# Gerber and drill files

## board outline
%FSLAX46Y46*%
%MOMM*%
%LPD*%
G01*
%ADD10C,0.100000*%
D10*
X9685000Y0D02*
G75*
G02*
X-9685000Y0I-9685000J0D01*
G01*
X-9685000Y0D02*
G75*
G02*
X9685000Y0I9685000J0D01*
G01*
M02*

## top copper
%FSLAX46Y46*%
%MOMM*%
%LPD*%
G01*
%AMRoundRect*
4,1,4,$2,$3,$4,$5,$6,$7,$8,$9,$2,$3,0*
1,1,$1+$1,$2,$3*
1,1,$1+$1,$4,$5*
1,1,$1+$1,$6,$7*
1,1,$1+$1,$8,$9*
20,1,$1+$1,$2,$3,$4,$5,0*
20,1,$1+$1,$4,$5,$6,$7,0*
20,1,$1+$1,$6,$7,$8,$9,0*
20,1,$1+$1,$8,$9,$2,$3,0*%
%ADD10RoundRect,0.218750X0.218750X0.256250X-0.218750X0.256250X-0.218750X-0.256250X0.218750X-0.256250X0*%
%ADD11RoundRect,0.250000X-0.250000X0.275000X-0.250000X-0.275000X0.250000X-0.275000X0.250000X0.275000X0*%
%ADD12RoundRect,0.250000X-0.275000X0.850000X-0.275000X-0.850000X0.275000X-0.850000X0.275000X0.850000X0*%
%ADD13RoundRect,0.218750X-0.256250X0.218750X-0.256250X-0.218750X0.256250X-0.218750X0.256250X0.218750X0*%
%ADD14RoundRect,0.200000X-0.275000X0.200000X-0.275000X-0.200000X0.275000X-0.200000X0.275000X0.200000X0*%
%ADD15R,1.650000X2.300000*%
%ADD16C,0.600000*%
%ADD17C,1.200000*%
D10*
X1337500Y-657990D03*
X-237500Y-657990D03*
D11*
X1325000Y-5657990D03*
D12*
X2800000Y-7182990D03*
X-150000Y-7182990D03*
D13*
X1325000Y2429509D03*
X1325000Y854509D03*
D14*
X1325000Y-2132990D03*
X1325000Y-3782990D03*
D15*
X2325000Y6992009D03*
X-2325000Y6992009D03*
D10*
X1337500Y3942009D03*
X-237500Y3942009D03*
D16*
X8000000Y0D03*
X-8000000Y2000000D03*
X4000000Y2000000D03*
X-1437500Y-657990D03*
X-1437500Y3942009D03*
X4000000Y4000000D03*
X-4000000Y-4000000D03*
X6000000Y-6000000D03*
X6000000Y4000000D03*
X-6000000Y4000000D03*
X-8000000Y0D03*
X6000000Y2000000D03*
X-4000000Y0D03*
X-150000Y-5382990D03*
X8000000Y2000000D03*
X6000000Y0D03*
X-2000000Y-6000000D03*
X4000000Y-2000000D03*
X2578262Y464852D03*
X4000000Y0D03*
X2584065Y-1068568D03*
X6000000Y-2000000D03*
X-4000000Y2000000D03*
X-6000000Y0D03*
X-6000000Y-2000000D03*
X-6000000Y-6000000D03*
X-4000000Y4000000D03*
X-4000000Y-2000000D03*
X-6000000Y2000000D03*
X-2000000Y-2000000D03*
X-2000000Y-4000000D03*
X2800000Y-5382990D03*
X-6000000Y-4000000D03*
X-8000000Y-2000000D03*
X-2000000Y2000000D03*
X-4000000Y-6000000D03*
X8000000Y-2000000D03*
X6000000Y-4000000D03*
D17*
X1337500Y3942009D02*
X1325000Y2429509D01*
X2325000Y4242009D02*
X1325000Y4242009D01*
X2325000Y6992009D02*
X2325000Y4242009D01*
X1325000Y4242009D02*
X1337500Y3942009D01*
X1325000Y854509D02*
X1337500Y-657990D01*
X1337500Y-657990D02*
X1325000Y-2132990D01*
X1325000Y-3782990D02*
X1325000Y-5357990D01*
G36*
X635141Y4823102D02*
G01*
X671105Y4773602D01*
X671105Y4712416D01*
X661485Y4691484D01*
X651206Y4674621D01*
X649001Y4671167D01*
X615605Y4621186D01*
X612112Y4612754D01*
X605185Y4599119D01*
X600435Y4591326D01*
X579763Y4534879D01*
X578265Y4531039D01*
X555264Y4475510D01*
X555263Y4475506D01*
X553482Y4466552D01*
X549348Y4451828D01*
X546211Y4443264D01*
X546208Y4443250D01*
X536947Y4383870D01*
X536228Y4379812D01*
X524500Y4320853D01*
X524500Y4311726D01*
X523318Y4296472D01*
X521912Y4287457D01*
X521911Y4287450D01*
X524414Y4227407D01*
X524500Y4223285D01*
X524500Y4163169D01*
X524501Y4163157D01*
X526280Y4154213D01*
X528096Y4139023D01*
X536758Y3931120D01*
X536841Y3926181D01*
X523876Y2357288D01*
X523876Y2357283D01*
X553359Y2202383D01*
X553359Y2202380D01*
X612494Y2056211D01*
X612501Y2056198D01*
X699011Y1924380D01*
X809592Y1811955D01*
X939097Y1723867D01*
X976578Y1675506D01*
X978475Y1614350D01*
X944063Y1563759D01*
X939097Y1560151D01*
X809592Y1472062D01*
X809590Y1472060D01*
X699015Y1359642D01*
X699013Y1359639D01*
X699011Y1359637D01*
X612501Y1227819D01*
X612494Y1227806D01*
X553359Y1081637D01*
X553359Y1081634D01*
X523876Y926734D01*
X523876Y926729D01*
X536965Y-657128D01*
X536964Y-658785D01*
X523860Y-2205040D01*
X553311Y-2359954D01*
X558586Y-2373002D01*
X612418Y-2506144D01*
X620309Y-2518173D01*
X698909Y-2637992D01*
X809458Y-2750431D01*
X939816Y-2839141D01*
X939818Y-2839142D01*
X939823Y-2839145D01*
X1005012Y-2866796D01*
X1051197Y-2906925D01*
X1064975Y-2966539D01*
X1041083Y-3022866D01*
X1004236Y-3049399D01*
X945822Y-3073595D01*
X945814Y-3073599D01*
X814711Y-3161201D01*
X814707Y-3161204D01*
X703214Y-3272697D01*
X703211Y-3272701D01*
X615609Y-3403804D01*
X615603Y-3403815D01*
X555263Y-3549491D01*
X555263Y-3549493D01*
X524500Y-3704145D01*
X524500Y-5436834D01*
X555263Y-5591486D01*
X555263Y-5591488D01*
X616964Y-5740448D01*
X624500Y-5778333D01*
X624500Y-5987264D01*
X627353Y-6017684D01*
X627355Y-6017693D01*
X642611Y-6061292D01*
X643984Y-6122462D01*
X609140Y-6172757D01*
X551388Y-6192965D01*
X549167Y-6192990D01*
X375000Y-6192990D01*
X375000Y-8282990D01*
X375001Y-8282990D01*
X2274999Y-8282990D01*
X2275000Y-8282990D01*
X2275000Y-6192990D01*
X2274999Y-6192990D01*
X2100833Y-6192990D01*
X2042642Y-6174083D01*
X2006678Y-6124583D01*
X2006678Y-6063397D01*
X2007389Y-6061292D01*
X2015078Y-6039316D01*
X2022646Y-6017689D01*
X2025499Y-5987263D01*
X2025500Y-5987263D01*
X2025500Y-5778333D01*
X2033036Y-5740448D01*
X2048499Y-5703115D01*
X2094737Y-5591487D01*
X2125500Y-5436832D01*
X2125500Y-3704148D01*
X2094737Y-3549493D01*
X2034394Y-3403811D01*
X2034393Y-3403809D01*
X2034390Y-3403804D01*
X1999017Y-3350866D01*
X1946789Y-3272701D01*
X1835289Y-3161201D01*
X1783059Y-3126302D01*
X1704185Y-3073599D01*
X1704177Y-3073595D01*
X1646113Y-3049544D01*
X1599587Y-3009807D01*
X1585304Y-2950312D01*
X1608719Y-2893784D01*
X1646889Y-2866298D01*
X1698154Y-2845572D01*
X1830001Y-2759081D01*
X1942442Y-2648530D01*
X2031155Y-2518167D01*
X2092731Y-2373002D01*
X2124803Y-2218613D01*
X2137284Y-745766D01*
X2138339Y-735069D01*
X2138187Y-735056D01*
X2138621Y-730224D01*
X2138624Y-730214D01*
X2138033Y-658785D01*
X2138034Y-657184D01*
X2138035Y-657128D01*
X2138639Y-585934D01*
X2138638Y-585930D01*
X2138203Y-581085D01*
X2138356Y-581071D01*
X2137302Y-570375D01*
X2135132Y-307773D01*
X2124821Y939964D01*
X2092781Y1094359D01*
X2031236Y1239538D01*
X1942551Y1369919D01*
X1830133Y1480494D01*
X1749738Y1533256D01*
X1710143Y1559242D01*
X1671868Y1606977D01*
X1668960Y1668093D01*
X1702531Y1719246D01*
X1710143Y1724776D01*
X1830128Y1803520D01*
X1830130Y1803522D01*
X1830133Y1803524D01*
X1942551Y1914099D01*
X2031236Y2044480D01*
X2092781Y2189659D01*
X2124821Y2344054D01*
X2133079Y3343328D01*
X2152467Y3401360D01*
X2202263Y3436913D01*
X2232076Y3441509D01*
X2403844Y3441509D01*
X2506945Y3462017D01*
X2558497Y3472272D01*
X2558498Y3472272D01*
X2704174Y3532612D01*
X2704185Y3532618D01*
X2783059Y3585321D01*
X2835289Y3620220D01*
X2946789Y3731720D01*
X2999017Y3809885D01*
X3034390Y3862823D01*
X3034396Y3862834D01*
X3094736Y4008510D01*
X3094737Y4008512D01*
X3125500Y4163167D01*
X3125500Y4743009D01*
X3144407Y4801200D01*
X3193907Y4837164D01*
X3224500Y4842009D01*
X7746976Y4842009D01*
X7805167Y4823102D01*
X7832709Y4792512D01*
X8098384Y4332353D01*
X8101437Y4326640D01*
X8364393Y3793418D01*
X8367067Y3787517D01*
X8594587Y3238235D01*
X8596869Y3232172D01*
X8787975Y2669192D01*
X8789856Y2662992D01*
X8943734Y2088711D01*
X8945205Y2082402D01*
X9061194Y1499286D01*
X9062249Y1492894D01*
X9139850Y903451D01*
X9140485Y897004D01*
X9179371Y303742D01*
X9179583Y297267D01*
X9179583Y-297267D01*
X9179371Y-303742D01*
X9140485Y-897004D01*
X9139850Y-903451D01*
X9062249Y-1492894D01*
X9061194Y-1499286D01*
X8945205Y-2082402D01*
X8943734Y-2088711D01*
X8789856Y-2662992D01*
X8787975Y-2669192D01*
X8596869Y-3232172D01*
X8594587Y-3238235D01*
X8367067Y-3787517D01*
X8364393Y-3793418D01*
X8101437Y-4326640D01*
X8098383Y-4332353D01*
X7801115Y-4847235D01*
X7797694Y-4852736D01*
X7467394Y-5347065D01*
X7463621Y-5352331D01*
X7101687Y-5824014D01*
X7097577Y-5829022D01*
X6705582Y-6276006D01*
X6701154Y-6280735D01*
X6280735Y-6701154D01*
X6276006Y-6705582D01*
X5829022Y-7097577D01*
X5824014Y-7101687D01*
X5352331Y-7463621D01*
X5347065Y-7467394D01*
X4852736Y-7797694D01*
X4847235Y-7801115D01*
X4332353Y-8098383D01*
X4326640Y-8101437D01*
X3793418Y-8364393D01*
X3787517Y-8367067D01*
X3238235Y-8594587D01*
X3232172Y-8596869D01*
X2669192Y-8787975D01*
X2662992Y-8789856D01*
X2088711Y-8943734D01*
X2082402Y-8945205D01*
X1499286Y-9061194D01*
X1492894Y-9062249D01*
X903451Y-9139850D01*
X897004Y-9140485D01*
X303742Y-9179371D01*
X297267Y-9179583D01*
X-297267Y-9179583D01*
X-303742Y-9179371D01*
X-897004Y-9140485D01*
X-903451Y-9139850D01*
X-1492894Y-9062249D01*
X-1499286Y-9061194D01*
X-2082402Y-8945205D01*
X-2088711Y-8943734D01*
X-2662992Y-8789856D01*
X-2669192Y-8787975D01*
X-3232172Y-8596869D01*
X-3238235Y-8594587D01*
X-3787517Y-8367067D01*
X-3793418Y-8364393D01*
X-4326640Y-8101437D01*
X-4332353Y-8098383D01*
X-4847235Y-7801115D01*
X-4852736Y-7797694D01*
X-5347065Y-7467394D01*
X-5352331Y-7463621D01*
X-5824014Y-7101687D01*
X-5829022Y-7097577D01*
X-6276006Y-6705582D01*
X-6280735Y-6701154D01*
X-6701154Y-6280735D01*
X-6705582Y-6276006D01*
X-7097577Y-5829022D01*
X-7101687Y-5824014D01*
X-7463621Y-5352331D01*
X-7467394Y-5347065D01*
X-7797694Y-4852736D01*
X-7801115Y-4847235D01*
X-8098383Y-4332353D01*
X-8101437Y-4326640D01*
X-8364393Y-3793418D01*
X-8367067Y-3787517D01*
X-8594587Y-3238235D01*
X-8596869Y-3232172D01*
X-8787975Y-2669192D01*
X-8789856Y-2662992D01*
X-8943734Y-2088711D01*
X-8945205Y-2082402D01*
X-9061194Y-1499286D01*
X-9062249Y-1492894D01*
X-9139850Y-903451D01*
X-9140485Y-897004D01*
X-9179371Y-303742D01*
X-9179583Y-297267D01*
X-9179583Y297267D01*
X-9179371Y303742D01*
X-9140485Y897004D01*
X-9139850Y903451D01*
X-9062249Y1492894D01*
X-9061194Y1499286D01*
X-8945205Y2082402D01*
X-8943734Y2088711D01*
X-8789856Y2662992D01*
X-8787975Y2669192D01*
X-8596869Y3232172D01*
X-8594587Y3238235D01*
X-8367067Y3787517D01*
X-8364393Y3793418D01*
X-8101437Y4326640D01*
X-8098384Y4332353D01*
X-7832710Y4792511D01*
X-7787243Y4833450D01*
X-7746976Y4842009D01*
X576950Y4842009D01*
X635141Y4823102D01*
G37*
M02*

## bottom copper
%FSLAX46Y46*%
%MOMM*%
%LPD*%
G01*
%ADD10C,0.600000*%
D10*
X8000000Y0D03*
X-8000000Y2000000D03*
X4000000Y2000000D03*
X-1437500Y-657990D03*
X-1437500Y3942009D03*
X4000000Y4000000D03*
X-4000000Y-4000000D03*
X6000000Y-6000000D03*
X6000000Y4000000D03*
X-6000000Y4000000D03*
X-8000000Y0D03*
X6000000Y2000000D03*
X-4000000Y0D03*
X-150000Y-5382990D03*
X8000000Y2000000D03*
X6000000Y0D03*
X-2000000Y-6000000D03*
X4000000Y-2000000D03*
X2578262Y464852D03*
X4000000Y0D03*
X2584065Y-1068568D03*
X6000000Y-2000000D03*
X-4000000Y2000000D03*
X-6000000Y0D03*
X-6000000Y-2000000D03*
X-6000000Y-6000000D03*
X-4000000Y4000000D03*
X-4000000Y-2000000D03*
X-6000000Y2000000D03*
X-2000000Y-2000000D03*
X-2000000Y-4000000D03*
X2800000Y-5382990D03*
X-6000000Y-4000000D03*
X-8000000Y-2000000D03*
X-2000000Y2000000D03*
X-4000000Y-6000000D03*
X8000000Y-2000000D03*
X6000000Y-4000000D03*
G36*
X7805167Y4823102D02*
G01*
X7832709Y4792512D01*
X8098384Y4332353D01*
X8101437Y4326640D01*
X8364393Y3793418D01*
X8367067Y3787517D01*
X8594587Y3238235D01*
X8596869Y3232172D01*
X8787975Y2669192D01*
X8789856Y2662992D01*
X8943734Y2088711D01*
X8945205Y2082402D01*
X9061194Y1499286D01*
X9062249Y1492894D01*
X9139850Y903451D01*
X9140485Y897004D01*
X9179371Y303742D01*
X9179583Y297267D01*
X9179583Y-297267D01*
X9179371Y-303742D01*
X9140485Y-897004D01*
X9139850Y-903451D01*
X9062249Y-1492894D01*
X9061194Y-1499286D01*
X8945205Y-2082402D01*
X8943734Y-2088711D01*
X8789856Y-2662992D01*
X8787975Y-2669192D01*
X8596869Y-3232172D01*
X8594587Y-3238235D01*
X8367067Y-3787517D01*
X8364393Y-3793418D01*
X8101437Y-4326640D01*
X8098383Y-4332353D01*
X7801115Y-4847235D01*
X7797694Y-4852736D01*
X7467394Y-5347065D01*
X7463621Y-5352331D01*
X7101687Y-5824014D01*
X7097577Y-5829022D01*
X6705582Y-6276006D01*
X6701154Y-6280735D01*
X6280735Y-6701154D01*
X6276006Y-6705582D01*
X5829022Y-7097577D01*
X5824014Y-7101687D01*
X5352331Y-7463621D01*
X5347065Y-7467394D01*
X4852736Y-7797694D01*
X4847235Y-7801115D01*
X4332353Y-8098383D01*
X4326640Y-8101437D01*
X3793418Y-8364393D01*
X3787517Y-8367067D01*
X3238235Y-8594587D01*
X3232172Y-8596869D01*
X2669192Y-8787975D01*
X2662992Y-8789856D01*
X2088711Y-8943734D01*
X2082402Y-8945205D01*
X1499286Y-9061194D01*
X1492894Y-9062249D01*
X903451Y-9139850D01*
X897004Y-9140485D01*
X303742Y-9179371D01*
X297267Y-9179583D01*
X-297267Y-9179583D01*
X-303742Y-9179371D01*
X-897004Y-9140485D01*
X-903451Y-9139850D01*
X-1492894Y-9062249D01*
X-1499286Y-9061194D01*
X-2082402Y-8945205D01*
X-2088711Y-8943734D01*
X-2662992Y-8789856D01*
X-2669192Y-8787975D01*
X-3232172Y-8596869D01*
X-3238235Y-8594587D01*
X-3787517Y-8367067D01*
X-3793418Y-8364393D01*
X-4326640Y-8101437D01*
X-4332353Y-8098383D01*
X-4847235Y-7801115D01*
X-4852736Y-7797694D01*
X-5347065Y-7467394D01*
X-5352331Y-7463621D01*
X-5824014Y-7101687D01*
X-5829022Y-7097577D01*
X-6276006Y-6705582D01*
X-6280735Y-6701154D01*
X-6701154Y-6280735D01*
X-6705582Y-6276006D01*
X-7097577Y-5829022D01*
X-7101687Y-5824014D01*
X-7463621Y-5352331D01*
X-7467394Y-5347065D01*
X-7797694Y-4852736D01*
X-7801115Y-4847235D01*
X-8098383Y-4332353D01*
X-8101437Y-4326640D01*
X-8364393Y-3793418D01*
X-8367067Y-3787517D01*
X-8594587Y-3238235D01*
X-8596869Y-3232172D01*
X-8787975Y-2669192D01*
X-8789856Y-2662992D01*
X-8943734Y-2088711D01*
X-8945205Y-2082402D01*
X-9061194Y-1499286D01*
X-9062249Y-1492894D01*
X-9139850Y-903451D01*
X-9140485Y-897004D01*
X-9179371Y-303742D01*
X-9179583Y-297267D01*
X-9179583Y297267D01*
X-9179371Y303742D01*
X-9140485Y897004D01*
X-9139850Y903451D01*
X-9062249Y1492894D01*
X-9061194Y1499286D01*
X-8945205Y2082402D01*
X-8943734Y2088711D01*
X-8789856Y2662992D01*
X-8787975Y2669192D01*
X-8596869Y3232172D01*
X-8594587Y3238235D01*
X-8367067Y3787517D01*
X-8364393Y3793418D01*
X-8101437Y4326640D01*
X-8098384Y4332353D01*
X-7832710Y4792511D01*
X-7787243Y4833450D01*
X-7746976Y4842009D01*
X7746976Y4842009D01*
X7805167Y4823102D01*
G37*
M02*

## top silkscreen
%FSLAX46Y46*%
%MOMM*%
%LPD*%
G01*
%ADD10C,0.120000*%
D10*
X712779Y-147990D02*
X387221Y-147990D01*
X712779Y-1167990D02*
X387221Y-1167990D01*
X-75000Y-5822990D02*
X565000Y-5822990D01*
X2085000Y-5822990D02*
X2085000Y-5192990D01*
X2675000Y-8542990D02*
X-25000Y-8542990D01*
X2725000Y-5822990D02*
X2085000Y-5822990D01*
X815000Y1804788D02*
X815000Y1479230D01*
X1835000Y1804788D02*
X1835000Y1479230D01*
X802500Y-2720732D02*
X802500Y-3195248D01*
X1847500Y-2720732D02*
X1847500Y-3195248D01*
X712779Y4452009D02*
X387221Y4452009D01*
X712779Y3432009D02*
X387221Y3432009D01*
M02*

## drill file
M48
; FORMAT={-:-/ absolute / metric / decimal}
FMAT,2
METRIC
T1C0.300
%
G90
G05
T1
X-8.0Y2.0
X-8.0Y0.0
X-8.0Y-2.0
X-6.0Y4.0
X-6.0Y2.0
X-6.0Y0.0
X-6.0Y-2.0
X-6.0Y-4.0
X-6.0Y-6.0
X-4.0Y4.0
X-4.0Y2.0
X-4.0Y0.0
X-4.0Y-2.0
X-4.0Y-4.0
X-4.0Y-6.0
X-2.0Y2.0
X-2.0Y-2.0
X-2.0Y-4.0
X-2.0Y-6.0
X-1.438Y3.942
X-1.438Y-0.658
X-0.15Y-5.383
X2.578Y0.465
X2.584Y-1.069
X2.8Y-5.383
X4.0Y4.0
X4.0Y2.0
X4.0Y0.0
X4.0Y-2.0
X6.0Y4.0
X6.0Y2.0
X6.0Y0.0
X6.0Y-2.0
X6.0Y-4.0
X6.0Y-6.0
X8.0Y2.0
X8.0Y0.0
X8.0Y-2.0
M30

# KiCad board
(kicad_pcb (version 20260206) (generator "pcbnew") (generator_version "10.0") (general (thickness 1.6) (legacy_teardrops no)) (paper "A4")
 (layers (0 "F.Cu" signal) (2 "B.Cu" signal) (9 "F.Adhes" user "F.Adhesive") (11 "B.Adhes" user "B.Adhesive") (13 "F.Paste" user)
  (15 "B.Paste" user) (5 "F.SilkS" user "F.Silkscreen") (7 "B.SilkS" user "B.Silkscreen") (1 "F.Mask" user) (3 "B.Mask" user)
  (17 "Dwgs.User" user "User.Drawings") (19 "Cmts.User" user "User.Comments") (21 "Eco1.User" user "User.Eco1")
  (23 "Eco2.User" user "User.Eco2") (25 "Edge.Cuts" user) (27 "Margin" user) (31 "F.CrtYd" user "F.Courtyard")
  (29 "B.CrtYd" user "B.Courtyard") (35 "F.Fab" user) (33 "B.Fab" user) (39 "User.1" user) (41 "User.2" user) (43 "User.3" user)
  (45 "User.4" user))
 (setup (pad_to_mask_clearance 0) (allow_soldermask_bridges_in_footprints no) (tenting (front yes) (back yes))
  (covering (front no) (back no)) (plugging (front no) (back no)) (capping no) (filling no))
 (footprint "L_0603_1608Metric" (layer "F.Cu") (at 0.55 0.65799 180)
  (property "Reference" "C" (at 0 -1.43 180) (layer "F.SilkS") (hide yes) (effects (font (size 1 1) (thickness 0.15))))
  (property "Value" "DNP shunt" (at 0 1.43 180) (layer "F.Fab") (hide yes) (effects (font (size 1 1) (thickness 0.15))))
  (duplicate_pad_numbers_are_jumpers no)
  (fp_line (start -0.162779 0.51) (end 0.162779 0.51) (stroke (width 0.12) (type solid)) (layer "F.SilkS"))
  (fp_line (start -0.162779 -0.51) (end 0.162779 -0.51) (stroke (width 0.12) (type solid)) (layer "F.SilkS"))
  (pad "1" smd roundrect (at -0.7875 0 180) (size 0.875 0.95) (layers "F.Cu" "F.Mask" "F.Paste") (roundrect_rratio 0.25) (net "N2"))
  (pad "2" smd roundrect (at 0.7875 0 180) (size 0.875 0.95) (layers "F.Cu" "F.Mask" "F.Paste") (roundrect_rratio 0.25) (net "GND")))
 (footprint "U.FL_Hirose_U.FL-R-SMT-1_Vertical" (layer "F.Cu") (at 1.325 7.18299 -90)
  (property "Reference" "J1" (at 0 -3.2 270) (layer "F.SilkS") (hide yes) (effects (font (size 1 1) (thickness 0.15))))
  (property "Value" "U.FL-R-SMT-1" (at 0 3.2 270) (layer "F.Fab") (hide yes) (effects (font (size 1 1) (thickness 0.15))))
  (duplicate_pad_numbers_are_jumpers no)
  (fp_line (start -1.36 1.4) (end -1.36 0.76) (stroke (width 0.12) (type solid)) (layer "F.SilkS"))
  (fp_line (start -1.36 -0.76) (end -1.99 -0.76) (stroke (width 0.12) (type solid)) (layer "F.SilkS"))
  (fp_line (start 1.36 -1.35) (end 1.36 1.35) (stroke (width 0.12) (type solid)) (layer "F.SilkS"))
  (fp_line (start -1.36 -1.4) (end -1.36 -0.76) (stroke (width 0.12) (type solid)) (layer "F.SilkS"))
  (pad "1" smd roundrect (at -1.525 0 270) (size 1.05 1) (layers "F.Cu" "F.Mask" "F.Paste") (roundrect_rratio 0.25) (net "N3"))
  (pad "2" smd roundrect (at 0 -1.475 270) (size 2.2 1.05) (layers "F.Cu" "F.Mask" "F.Paste") (roundrect_rratio 0.2380952381) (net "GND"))
  (pad "2" smd roundrect (at 0 1.475 270) (size 2.2 1.05) (layers "F.Cu" "F.Mask" "F.Paste") (roundrect_rratio 0.2380952381) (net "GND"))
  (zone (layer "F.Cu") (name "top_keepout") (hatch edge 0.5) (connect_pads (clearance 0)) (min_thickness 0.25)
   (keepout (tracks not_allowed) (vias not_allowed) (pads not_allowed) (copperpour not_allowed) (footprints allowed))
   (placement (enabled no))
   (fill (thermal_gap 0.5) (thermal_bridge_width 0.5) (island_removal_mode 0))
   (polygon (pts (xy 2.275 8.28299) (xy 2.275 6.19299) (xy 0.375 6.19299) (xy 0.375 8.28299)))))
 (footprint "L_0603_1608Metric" (layer "F.Cu") (at 1.325 -1.642009 -90)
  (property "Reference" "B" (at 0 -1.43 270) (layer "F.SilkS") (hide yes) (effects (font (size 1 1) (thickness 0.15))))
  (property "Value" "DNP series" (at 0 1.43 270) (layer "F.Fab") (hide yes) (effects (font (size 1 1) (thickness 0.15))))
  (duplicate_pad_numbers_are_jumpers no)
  (fp_line (start -0.162779 0.51) (end 0.162779 0.51) (stroke (width 0.12) (type solid)) (layer "F.SilkS"))
  (fp_line (start -0.162779 -0.51) (end 0.162779 -0.51) (stroke (width 0.12) (type solid)) (layer "F.SilkS"))
  (pad "1" smd roundrect (at -0.7875 0 270) (size 0.875 0.95) (layers "F.Cu" "F.Mask" "F.Paste") (roundrect_rratio 0.25) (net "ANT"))
  (pad "2" smd roundrect (at 0.7875 0 270) (size 0.875 0.95) (layers "F.Cu" "F.Mask" "F.Paste") (roundrect_rratio 0.25) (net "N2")))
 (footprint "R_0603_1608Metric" (layer "F.Cu") (at 1.325 2.95799 -90)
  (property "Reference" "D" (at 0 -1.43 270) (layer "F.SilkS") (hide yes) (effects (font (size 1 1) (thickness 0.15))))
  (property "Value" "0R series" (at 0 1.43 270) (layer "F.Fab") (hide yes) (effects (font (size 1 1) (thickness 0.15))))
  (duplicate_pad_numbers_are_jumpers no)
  (fp_line (start -0.237258 0.5225) (end 0.237258 0.5225) (stroke (width 0.12) (type solid)) (layer "F.SilkS"))
  (fp_line (start -0.237258 -0.5225) (end 0.237258 -0.5225) (stroke (width 0.12) (type solid)) (layer "F.SilkS"))
  (pad "1" smd roundrect (at -0.825 0 270) (size 0.8 0.95) (layers "F.Cu" "F.Mask" "F.Paste") (roundrect_rratio 0.25) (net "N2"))
  (pad "2" smd roundrect (at 0.825 0 270) (size 0.8 0.95) (layers "F.Cu" "F.Mask" "F.Paste") (roundrect_rratio 0.25) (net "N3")))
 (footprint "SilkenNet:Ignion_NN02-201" (layer "F.Cu") (at 0 -6.992009)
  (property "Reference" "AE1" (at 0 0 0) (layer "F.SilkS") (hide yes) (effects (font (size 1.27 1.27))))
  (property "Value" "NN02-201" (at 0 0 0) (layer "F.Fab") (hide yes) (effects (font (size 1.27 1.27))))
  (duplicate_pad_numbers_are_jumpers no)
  (pad "1" smd rect (at 2.325 0) (size 1.65 2.3) (layers "F.Cu" "F.Mask" "F.Paste") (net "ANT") (thermal_bridge_angle 45))
  (pad "2" smd rect (at -2.325 0) (size 1.65 2.3) (layers "F.Cu" "F.Mask" "F.Paste") (thermal_bridge_angle 45)))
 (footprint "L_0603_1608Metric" (layer "F.Cu") (at 0.55 -3.942009 180)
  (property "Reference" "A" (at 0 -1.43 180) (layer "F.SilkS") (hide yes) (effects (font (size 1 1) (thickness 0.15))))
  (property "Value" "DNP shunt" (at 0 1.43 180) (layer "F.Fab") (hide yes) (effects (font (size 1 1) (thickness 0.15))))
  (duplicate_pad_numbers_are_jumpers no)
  (fp_line (start -0.162779 0.51) (end 0.162779 0.51) (stroke (width 0.12) (type solid)) (layer "F.SilkS"))
  (fp_line (start -0.162779 -0.51) (end 0.162779 -0.51) (stroke (width 0.12) (type solid)) (layer "F.SilkS"))
  (pad "1" smd roundrect (at -0.7875 0 180) (size 0.875 0.95) (layers "F.Cu" "F.Mask" "F.Paste") (roundrect_rratio 0.25) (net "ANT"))
  (pad "2" smd roundrect (at 0.7875 0 180) (size 0.875 0.95) (layers "F.Cu" "F.Mask" "F.Paste") (roundrect_rratio 0.25) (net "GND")))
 (gr_circle (center 0 0) (end 9.685 0) (stroke (width 0.1) (type default)) (fill no) (layer "Edge.Cuts"))
 (via (at 8 0) (size 0.6) (drill 0.3) (layers "F.Cu" "B.Cu") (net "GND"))
 (via (at -8 -2) (size 0.6) (drill 0.3) (layers "F.Cu" "B.Cu") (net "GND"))
 (via (at 4 -2) (size 0.6) (drill 0.3) (layers "F.Cu" "B.Cu") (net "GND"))
 (via (at -1.4375 0.65799) (size 0.6) (drill 0.3) (layers "F.Cu" "B.Cu") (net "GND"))
 (via (at -1.4375 -3.942009) (size 0.6) (drill 0.3) (layers "F.Cu" "B.Cu") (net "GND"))
 (via (at 4 -4) (size 0.6) (drill 0.3) (layers "F.Cu" "B.Cu") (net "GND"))
 (via (at -4 4) (size 0.6) (drill 0.3) (layers "F.Cu" "B.Cu") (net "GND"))
 (via (at 6 6) (size 0.6) (drill 0.3) (layers "F.Cu" "B.Cu") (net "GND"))
 (via (at 6 -4) (size 0.6) (drill 0.3) (layers "F.Cu" "B.Cu") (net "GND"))
 (via (at -6 -4) (size 0.6) (drill 0.3) (layers "F.Cu" "B.Cu") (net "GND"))
 (via (at -8 0) (size 0.6) (drill 0.3) (layers "F.Cu" "B.Cu") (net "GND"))
 (via (at 6 -2) (size 0.6) (drill 0.3) (layers "F.Cu" "B.Cu") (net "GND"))
 (via (at -4 0) (size 0.6) (drill 0.3) (layers "F.Cu" "B.Cu") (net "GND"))
 (via (at -0.15 5.38299) (size 0.6) (drill 0.3) (layers "F.Cu" "B.Cu") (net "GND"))
 (via (at 8 -2) (size 0.6) (drill 0.3) (layers "F.Cu" "B.Cu") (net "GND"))
 (via (at 6 0) (size 0.6) (drill 0.3) (layers "F.Cu" "B.Cu") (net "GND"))
 (via (at -2 6) (size 0.6) (drill 0.3) (layers "F.Cu" "B.Cu") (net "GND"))
 (via (at 4 2) (size 0.6) (drill 0.3) (layers "F.Cu" "B.Cu") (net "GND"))
 (via (at 2.578262 -0.464852) (size 0.6) (drill 0.3) (layers "F.Cu" "B.Cu") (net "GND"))
 (via (at 4 0) (size 0.6) (drill 0.3) (layers "F.Cu" "B.Cu") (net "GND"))
 (via (at 2.584065 1.068568) (size 0.6) (drill 0.3) (layers "F.Cu" "B.Cu") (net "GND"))
 (via (at 6 2) (size 0.6) (drill 0.3) (layers "F.Cu" "B.Cu") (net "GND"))
 (via (at -4 -2) (size 0.6) (drill 0.3) (layers "F.Cu" "B.Cu") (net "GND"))
 (via (at -6 0) (size 0.6) (drill 0.3) (layers "F.Cu" "B.Cu") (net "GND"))
 (via (at -6 2) (size 0.6) (drill 0.3) (layers "F.Cu" "B.Cu") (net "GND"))
 (via (at -6 6) (size 0.6) (drill 0.3) (layers "F.Cu" "B.Cu") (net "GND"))
 (via (at -4 -4) (size 0.6) (drill 0.3) (layers "F.Cu" "B.Cu") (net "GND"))
 (via (at -4 2) (size 0.6) (drill 0.3) (layers "F.Cu" "B.Cu") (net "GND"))
 (via (at -6 -2) (size 0.6) (drill 0.3) (layers "F.Cu" "B.Cu") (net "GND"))
 (via (at -2 2) (size 0.6) (drill 0.3) (layers "F.Cu" "B.Cu") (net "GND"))
 (via (at -2 4) (size 0.6) (drill 0.3) (layers "F.Cu" "B.Cu") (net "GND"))
 (via (at 2.8 5.38299) (size 0.6) (drill 0.3) (layers "F.Cu" "B.Cu") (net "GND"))
 (via (at -6 4) (size 0.6) (drill 0.3) (layers "F.Cu" "B.Cu") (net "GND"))
 (via (at -8 2) (size 0.6) (drill 0.3) (layers "F.Cu" "B.Cu") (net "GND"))
 (via (at -2 -2) (size 0.6) (drill 0.3) (layers "F.Cu" "B.Cu") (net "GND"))
 (via (at -4 6) (size 0.6) (drill 0.3) (layers "F.Cu" "B.Cu") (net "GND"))
 (via (at 8 2) (size 0.6) (drill 0.3) (layers "F.Cu" "B.Cu") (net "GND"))
 (via (at 6 4) (size 0.6) (drill 0.3) (layers "F.Cu" "B.Cu") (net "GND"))
 (segment (start 1.3375 -3.942009) (end 1.325 -2.429509) (width 1.2) (layer "F.Cu") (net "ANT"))
 (segment (start 2.325 -4.242009) (end 1.325 -4.242009) (width 1.2) (layer "F.Cu") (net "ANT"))
 (segment (start 2.325 -6.992009) (end 2.325 -4.242009) (width 1.2) (layer "F.Cu") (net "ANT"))
 (segment (start 1.325 -4.242009) (end 1.3375 -3.942009) (width 1.2) (layer "F.Cu") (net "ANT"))
 (segment (start 1.325 -0.854509) (end 1.3375 0.65799) (width 1.2) (layer "F.Cu") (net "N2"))
 (segment (start 1.3375 0.65799) (end 1.325 2.13299) (width 1.2) (layer "F.Cu") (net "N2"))
 (segment (start 1.325 3.78299) (end 1.325 5.35799) (width 1.2) (layer "F.Cu") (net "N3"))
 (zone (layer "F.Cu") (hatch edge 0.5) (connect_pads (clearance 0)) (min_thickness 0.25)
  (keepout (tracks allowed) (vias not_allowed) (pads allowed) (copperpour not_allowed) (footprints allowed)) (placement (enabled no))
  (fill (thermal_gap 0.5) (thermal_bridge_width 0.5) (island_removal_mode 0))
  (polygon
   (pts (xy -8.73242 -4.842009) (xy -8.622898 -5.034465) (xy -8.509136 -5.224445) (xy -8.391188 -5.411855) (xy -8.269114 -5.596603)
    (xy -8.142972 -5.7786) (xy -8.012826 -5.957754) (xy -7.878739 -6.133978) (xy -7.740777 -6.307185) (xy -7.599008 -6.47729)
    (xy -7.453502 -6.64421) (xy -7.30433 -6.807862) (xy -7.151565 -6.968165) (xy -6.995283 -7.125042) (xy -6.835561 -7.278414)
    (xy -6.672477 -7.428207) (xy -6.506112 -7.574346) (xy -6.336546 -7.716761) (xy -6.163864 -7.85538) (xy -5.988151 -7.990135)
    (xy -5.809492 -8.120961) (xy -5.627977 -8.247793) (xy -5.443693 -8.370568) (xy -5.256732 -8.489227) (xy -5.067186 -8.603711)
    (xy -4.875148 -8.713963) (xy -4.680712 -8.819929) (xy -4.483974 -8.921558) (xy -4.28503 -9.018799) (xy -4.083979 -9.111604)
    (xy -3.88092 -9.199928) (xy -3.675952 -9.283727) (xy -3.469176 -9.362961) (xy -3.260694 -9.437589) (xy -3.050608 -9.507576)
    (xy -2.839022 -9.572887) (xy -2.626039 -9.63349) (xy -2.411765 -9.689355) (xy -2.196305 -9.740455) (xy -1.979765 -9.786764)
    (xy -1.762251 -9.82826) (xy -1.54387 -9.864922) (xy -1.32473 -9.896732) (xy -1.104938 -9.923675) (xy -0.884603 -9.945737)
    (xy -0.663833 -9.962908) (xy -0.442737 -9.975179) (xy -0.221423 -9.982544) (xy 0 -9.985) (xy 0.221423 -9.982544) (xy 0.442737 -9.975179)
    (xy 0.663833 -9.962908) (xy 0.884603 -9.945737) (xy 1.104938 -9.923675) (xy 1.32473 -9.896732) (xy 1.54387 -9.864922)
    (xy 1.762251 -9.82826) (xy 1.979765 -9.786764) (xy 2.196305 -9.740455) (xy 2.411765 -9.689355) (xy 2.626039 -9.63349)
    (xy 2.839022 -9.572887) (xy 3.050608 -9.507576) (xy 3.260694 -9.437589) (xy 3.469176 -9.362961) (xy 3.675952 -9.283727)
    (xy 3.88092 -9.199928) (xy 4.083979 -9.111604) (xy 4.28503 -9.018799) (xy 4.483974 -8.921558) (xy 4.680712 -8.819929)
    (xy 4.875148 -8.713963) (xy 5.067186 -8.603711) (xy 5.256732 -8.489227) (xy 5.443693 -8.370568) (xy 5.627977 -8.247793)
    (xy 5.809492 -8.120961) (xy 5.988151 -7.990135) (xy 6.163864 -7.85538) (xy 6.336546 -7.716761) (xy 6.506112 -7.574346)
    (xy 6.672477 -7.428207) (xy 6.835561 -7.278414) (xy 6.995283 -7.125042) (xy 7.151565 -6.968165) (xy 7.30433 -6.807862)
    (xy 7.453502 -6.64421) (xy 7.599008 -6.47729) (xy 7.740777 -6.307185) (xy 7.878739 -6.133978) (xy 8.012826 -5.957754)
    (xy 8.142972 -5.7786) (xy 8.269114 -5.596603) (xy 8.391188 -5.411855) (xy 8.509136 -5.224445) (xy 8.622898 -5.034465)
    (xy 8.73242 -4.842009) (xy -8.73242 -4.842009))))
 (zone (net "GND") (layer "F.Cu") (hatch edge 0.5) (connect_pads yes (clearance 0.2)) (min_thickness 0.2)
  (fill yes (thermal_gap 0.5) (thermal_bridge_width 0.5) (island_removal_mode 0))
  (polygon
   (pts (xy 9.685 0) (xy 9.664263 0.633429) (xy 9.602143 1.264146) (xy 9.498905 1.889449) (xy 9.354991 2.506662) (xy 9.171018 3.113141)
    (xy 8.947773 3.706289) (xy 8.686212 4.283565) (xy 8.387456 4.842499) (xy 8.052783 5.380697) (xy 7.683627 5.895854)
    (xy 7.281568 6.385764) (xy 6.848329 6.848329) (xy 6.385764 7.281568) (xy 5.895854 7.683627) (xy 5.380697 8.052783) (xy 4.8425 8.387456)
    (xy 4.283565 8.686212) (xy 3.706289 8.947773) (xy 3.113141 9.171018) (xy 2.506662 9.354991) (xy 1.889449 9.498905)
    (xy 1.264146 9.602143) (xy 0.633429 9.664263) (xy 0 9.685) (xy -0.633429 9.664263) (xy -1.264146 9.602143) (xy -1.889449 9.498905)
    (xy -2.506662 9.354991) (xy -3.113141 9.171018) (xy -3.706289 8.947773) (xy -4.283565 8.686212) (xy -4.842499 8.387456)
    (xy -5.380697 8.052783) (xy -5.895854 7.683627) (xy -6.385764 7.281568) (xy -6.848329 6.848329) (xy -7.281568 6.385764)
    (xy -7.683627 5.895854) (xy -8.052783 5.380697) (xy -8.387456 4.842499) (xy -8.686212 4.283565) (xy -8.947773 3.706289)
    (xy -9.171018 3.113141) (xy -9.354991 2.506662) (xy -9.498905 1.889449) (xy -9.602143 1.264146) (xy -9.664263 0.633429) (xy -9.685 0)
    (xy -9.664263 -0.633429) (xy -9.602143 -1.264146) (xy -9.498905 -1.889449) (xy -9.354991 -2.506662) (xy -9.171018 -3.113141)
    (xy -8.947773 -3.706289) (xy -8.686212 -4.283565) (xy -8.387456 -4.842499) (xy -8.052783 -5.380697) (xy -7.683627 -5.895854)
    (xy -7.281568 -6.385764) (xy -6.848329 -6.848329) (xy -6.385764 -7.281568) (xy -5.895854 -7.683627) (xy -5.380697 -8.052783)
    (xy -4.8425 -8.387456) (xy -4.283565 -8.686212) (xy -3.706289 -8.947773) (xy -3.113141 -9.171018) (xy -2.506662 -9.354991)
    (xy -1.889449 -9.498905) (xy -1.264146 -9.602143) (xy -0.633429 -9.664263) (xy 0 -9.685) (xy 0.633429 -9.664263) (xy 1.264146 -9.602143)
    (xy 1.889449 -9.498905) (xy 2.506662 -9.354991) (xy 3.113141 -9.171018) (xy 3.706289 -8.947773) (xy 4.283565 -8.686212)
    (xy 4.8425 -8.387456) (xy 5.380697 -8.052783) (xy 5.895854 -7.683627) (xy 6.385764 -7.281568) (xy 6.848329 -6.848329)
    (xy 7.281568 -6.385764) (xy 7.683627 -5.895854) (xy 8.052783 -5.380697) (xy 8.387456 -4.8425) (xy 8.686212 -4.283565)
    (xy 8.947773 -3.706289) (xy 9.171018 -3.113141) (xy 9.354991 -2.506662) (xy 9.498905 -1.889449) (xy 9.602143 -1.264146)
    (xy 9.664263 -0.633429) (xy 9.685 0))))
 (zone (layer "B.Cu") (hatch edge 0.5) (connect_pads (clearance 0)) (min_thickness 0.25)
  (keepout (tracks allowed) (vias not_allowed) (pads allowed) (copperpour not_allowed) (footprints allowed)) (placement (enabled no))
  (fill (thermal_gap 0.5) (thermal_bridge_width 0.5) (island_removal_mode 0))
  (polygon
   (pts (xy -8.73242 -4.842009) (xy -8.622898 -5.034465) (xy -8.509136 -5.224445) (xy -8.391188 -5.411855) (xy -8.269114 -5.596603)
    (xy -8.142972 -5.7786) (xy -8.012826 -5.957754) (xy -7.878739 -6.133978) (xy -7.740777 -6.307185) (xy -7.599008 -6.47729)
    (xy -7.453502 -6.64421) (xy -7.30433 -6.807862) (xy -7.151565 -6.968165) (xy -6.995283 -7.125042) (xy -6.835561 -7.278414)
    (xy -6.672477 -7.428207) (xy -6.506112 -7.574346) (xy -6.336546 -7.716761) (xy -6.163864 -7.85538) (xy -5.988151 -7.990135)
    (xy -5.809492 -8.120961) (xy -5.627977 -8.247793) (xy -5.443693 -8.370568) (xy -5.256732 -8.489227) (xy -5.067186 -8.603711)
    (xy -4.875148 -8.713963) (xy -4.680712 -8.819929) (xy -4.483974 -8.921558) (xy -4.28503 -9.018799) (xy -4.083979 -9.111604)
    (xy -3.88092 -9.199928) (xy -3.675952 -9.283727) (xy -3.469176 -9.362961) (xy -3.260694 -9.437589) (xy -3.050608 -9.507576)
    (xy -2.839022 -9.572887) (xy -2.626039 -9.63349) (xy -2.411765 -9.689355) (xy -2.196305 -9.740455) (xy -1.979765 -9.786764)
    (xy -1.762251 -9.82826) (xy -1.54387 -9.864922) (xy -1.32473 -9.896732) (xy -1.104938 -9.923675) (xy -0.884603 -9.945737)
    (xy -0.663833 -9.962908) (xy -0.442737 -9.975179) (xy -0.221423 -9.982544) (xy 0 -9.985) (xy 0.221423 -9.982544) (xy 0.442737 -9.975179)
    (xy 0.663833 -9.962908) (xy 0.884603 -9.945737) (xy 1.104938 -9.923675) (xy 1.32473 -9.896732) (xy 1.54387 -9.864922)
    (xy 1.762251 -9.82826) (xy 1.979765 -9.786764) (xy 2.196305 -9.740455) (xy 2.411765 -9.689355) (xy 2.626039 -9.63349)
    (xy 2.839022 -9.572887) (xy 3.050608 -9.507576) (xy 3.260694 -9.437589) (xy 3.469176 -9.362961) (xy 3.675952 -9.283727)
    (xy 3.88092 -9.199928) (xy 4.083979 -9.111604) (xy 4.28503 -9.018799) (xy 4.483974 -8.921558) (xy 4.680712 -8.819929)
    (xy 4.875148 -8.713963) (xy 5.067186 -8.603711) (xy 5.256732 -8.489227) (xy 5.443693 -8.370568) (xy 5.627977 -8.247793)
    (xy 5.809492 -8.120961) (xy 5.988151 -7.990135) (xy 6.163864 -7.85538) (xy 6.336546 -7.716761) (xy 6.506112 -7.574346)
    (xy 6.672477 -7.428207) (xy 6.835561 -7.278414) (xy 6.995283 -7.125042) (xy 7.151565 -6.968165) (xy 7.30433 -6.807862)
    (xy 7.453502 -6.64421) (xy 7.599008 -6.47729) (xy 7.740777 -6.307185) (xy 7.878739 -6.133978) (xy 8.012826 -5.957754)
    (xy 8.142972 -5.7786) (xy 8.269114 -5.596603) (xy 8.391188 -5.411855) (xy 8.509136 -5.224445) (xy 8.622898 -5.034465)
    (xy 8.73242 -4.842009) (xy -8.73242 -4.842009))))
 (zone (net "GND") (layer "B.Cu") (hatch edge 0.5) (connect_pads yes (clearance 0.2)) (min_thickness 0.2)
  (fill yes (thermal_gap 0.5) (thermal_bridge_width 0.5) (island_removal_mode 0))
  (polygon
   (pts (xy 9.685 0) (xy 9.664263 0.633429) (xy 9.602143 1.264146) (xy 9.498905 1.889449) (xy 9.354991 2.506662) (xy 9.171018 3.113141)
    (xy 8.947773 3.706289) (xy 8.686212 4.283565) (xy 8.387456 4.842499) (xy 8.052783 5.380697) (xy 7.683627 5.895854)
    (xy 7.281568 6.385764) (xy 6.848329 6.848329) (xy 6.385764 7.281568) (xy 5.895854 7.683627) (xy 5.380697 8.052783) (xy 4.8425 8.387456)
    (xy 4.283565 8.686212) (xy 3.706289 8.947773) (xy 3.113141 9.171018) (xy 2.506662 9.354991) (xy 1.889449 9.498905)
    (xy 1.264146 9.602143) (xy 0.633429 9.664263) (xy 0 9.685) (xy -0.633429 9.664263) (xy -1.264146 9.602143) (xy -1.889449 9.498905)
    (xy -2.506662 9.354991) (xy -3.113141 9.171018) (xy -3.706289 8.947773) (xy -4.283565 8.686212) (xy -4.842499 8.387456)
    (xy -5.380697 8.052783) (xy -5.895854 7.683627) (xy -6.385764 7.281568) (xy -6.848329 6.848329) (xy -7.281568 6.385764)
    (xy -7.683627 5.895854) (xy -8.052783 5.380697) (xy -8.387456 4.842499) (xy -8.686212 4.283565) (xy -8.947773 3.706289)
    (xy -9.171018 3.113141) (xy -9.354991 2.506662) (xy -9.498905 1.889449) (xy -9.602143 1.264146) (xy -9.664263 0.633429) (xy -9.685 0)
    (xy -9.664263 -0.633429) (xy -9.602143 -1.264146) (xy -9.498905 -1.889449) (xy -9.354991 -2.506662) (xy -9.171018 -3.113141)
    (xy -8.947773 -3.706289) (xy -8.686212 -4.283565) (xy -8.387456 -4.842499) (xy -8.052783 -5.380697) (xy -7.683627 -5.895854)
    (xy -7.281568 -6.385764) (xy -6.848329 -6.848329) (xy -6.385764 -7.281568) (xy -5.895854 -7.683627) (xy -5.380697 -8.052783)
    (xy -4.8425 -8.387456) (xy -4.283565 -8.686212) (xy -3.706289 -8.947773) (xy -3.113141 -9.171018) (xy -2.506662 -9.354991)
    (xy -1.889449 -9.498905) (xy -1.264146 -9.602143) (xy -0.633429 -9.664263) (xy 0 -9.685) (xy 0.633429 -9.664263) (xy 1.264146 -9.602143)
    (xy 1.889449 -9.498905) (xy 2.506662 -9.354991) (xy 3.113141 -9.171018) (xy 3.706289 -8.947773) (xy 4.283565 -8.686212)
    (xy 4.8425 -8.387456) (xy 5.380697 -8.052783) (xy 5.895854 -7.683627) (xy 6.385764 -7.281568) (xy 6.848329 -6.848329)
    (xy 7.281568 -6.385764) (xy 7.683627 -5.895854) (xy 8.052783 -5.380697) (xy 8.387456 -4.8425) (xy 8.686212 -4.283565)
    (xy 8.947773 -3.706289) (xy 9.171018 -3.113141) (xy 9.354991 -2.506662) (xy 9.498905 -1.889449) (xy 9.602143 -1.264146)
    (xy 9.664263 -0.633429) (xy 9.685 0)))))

